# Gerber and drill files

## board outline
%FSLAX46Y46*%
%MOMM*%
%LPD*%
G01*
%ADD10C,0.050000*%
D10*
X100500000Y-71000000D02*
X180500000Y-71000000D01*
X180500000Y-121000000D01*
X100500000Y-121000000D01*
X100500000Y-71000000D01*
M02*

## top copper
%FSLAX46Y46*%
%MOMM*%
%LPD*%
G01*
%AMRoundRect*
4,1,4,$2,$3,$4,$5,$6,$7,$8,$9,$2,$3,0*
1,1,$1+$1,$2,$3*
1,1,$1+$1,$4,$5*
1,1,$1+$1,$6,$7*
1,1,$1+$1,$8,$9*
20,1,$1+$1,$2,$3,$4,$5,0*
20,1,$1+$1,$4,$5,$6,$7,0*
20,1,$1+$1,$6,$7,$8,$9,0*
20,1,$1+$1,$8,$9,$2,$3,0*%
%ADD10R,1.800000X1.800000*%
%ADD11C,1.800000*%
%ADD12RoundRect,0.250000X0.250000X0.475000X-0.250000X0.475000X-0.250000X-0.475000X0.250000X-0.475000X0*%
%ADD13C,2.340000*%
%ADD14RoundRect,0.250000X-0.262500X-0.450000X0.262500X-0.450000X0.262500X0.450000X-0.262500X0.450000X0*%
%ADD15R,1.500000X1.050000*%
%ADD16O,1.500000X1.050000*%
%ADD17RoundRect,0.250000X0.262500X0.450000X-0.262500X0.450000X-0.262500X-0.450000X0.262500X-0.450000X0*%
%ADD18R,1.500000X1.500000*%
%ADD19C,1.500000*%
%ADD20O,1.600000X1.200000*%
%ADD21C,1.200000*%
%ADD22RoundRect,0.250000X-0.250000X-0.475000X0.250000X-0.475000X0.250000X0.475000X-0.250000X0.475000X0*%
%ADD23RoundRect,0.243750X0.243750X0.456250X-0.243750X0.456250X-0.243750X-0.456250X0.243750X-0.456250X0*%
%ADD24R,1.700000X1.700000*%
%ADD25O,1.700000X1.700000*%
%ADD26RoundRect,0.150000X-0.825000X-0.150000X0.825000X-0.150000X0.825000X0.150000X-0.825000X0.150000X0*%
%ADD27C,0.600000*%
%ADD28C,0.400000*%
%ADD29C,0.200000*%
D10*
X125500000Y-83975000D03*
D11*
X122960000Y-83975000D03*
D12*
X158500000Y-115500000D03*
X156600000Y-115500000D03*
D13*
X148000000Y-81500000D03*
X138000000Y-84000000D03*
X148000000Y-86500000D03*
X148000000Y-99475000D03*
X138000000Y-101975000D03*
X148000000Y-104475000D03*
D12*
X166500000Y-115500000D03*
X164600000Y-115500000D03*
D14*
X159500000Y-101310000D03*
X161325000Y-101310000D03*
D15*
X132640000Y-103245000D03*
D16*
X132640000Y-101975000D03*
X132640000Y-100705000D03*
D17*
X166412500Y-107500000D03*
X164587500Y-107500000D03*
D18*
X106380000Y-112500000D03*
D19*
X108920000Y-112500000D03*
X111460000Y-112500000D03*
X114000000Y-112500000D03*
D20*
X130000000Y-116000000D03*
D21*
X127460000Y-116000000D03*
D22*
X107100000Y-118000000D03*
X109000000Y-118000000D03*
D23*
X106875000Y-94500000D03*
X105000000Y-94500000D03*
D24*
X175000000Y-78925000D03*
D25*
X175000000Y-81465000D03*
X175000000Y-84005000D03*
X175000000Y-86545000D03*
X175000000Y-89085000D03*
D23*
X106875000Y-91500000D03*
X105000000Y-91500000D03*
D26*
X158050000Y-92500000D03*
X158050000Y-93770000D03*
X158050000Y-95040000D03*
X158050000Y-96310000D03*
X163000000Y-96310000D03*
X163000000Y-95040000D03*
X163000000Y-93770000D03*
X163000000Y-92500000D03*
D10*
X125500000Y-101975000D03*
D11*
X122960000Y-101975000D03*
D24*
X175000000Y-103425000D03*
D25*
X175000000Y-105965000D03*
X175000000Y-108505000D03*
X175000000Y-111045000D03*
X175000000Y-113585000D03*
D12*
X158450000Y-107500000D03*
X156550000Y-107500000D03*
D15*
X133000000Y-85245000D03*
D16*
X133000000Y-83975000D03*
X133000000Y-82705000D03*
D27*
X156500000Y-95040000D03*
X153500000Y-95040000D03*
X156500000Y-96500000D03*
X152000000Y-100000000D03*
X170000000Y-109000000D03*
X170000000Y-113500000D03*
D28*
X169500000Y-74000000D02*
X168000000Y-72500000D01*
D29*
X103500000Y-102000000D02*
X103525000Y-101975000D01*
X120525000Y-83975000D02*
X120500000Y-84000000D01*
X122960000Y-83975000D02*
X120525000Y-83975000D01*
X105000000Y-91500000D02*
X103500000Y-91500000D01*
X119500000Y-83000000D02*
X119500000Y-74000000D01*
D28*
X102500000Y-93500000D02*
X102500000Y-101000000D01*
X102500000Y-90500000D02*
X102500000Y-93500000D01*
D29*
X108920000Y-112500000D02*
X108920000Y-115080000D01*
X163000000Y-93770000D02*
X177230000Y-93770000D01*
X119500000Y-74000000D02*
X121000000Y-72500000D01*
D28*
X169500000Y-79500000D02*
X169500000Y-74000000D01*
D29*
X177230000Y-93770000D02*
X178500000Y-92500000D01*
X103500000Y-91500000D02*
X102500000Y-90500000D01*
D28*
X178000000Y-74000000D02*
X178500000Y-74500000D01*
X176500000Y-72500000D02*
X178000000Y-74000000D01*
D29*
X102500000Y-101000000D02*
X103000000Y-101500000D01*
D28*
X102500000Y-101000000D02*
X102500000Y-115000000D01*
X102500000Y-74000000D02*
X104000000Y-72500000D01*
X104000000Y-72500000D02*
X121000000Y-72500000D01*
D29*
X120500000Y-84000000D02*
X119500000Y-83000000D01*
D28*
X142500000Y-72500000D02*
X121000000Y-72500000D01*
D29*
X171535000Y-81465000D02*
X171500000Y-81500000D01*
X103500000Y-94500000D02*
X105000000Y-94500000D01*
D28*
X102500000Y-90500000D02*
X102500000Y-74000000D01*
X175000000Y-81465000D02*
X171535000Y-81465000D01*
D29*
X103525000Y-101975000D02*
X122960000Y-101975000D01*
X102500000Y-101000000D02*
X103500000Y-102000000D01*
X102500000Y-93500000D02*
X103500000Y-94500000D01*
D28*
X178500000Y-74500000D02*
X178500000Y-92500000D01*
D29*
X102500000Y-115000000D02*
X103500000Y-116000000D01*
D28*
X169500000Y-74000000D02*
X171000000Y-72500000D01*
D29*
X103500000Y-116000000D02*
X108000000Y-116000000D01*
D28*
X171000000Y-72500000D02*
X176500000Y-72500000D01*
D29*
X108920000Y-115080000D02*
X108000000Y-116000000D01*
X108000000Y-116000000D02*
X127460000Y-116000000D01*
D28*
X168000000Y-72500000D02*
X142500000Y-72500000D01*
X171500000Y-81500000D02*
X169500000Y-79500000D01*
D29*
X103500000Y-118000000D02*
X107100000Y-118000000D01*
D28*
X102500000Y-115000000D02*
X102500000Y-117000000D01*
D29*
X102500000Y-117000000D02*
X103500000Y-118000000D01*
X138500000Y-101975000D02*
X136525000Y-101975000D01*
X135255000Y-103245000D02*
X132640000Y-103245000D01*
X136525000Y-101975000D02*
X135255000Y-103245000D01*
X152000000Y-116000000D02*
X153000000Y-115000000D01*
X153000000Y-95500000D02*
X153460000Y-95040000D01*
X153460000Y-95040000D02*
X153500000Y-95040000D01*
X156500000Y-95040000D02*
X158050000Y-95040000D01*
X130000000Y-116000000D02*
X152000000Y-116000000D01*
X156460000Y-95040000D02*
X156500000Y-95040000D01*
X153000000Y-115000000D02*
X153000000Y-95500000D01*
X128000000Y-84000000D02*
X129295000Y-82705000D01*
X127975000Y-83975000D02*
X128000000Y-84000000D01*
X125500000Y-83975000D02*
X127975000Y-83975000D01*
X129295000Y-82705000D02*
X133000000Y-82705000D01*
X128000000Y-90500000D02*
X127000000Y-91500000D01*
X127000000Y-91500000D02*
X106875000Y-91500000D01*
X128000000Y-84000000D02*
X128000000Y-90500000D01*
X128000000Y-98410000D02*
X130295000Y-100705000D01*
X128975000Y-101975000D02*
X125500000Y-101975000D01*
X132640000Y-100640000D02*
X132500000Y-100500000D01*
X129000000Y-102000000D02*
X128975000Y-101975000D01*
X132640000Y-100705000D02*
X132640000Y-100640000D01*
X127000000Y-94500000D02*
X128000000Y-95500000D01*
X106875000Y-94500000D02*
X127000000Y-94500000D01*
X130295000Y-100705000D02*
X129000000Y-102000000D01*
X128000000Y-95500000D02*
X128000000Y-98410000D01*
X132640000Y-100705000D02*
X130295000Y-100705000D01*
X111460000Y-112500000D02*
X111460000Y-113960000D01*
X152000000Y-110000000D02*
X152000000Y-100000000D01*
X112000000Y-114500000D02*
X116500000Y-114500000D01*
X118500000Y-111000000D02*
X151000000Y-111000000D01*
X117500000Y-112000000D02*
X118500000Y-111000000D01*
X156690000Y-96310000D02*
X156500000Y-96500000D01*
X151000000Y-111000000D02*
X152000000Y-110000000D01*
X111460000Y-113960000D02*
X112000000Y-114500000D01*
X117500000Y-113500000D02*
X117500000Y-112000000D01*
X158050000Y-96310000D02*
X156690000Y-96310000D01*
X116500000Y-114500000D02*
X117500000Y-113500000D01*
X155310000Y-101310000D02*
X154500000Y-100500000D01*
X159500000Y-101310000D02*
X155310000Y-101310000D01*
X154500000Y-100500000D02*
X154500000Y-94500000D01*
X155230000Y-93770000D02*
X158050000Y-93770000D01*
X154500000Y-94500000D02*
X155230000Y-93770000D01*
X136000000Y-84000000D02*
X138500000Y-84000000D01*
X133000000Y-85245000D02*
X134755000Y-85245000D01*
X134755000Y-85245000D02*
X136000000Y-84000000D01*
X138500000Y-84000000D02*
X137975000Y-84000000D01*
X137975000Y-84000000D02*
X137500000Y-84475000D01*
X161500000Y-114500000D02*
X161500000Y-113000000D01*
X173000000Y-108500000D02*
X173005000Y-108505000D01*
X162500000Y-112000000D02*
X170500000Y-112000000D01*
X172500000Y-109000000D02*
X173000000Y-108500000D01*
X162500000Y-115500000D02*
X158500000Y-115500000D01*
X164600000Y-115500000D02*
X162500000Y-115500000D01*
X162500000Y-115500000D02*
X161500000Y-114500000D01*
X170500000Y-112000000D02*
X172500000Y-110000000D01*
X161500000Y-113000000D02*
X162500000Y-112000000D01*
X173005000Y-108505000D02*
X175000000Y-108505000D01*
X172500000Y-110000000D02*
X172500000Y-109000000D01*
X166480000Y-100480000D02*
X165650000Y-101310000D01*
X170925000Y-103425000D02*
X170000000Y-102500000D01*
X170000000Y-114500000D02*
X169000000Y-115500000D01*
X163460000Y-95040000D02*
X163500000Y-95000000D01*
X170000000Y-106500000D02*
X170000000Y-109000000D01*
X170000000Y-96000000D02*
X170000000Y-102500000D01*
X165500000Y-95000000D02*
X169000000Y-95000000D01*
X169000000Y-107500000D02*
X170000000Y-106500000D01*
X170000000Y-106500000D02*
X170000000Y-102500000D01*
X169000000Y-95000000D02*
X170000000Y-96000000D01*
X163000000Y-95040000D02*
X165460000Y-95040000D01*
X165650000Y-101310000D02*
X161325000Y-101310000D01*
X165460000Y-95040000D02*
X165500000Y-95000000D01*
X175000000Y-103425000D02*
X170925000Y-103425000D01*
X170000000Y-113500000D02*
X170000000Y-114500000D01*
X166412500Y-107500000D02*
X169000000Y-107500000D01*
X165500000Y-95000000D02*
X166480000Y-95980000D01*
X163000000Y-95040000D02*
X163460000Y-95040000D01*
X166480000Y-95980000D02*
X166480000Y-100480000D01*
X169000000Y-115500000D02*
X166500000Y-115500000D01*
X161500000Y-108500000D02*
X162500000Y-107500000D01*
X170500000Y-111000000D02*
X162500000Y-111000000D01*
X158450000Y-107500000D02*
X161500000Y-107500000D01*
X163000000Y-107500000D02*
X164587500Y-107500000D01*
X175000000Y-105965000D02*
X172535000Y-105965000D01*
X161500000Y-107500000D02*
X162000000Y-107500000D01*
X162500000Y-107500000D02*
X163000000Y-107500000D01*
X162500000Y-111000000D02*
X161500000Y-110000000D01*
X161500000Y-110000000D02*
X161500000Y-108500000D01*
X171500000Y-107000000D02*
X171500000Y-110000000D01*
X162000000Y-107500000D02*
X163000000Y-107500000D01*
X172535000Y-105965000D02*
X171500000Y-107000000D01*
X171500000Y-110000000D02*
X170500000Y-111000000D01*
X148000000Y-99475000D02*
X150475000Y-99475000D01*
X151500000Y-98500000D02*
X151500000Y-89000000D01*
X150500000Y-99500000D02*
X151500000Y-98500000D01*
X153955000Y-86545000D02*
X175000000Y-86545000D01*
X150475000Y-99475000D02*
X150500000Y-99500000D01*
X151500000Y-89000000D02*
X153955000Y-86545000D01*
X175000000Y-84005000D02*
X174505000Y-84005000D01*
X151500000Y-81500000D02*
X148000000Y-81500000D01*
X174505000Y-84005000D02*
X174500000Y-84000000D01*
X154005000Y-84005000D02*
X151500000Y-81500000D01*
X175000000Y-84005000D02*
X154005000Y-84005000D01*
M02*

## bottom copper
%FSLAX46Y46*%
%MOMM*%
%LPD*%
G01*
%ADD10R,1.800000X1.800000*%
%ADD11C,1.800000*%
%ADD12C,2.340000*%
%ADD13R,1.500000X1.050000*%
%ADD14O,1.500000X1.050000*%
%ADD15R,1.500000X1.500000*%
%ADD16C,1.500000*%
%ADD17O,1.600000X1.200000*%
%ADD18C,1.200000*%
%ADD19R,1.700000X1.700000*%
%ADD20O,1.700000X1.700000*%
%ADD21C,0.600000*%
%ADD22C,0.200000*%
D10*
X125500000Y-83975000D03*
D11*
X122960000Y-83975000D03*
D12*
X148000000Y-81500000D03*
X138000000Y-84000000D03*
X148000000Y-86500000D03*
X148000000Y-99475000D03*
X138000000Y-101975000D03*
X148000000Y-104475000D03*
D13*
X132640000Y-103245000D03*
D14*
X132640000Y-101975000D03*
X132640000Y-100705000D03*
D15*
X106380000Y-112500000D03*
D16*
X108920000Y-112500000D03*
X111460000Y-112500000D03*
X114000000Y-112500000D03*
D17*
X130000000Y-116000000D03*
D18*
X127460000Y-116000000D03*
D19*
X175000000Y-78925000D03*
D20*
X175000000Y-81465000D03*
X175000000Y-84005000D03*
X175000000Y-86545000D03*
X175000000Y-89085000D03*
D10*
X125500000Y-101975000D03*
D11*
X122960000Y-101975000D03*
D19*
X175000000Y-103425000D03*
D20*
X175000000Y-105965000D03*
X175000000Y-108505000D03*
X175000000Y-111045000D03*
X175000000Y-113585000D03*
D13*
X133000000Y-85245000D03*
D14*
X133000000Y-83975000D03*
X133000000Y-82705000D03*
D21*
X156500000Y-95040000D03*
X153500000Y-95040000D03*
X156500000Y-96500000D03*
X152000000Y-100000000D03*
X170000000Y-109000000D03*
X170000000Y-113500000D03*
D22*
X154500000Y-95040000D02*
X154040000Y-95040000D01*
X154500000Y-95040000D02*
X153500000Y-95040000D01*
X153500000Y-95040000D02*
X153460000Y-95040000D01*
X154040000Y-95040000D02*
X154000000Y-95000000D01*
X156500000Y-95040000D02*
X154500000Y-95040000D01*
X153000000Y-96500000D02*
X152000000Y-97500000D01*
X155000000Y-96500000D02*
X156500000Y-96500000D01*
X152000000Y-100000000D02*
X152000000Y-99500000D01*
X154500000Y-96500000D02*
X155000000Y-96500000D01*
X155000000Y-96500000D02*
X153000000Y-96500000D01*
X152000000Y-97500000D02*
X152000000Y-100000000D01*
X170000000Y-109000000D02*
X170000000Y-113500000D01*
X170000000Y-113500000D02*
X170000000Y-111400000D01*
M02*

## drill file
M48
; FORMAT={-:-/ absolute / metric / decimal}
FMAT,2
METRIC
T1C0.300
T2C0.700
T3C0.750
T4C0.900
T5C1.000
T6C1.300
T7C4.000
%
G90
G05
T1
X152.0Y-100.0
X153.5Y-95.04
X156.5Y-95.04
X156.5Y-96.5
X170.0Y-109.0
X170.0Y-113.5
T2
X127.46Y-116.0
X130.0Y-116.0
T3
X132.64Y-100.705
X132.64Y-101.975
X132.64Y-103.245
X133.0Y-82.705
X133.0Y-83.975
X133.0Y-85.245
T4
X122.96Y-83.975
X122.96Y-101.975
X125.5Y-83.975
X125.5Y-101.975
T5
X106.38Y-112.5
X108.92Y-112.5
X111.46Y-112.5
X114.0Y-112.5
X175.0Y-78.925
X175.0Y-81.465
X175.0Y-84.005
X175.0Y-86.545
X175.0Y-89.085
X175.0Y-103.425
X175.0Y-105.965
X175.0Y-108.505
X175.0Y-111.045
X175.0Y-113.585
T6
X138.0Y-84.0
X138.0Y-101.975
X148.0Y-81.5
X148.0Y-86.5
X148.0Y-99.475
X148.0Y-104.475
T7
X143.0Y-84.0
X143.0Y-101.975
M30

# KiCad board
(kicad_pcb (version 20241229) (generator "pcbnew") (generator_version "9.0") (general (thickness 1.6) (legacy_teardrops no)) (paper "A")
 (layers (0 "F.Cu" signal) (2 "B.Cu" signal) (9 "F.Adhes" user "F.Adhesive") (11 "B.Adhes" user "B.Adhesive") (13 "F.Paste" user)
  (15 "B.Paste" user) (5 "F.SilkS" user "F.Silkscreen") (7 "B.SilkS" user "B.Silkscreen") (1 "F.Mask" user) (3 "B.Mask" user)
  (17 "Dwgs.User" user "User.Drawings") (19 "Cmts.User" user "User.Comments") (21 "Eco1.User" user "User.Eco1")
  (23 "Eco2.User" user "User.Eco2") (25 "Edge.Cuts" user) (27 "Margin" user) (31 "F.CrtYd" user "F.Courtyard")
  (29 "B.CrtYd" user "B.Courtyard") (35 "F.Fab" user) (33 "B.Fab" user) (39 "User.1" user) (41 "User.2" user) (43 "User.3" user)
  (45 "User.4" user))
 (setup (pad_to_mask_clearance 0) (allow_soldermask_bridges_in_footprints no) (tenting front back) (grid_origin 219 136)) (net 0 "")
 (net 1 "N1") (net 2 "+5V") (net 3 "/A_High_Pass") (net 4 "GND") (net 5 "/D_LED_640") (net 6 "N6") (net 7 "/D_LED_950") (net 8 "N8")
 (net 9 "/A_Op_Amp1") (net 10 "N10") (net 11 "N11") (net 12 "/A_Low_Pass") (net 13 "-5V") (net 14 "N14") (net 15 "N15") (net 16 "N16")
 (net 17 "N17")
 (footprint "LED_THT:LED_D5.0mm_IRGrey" (layer "F.Cu") (at 125.5 83.975 180)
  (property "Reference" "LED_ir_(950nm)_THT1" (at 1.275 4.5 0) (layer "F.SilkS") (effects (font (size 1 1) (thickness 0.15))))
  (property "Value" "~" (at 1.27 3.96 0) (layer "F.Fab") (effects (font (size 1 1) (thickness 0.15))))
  (pad "1" thru_hole rect (at 0 0 180) (size 1.8 1.8) (drill 0.9) (layers "*.Cu" "*.Mask") (remove_unused_layers no) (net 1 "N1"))
  (pad "2" thru_hole circle (at 2.54 0 180) (size 1.8 1.8) (drill 0.9) (layers "*.Cu" "*.Mask") (remove_unused_layers no) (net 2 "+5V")))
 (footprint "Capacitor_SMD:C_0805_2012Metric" (layer "F.Cu") (at 157.55 115.5 180)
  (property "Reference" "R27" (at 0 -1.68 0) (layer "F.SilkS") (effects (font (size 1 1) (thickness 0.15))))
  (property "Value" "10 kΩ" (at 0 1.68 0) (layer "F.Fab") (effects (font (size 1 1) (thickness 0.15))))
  (pad "1" smd roundrect (at -0.95 0 180) (size 1 1.45) (layers "F.Cu" "F.Mask" "F.Paste") (roundrect_rratio 0.25) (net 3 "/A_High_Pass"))
  (pad "2" smd roundrect (at 0.95 0 180) (size 1 1.45) (layers "F.Cu" "F.Mask" "F.Paste") (roundrect_rratio 0.25) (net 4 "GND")))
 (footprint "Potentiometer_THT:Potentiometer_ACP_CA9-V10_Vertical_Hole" (layer "F.Cu") (at 148 81.5 180)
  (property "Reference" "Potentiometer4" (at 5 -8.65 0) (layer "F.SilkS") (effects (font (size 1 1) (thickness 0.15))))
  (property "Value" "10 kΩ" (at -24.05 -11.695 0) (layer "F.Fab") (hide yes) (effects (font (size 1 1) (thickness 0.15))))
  (pad "" np_thru_hole circle (at 5 -2.5 180) (size 4 4) (drill 4) (layers "*.Cu" "*.Mask"))
  (pad "1" thru_hole circle (at 0 0 180) (size 2.34 2.34) (drill 1.3) (layers "*.Cu" "*.Mask") (remove_unused_layers no)
   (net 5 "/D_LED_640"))
  (pad "2" thru_hole circle (at 10 -2.5 180) (size 2.34 2.34) (drill 1.3) (layers "*.Cu" "*.Mask") (remove_unused_layers no) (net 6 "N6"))
  (pad "3" thru_hole circle (at 0 -5 180) (size 2.34 2.34) (drill 1.3) (layers "*.Cu" "*.Mask") (remove_unused_layers no) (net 4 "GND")))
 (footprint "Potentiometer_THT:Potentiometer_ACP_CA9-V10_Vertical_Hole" (layer "F.Cu") (at 148 99.475 180)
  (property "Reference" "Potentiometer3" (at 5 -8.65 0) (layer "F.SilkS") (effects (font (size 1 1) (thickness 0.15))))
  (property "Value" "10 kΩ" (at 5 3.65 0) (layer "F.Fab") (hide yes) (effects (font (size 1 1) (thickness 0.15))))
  (pad "" np_thru_hole circle (at 5 -2.5 180) (size 4 4) (drill 4) (layers "*.Cu" "*.Mask"))
  (pad "1" thru_hole circle (at 0 0 180) (size 2.34 2.34) (drill 1.3) (layers "*.Cu" "*.Mask") (remove_unused_layers no)
   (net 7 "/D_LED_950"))
  (pad "2" thru_hole circle (at 10 -2.5 180) (size 2.34 2.34) (drill 1.3) (layers "*.Cu" "*.Mask") (remove_unused_layers no) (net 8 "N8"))
  (pad "3" thru_hole circle (at 0 -5 180) (size 2.34 2.34) (drill 1.3) (layers "*.Cu" "*.Mask") (remove_unused_layers no) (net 4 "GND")))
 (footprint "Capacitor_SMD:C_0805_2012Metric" (layer "F.Cu") (at 165.55 115.5 180)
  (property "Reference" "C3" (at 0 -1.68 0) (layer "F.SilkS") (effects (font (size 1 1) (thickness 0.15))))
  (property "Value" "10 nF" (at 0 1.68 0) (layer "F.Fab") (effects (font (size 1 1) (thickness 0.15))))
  (pad "1" smd roundrect (at -0.95 0 180) (size 1 1.45) (layers "F.Cu" "F.Mask" "F.Paste") (roundrect_rratio 0.25) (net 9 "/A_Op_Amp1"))
  (pad "2" smd roundrect (at 0.95 0 180) (size 1 1.45) (layers "F.Cu" "F.Mask" "F.Paste") (roundrect_rratio 0.25) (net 3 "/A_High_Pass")))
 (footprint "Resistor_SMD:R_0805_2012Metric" (layer "F.Cu") (at 160.4125 101.31)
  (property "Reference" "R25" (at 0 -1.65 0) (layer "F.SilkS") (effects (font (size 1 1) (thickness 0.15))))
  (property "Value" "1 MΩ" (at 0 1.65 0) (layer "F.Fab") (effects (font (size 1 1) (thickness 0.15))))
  (pad "1" smd roundrect (at -0.9125 0) (size 1.025 1.4) (layers "F.Cu" "F.Mask" "F.Paste") (roundrect_rratio 0.243902) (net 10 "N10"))
  (pad "2" smd roundrect (at 0.9125 0) (size 1.025 1.4) (layers "F.Cu" "F.Mask" "F.Paste") (roundrect_rratio 0.243902) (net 9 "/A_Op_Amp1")))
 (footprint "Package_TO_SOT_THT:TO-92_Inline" (layer "F.Cu") (at 132.64 103.245 90)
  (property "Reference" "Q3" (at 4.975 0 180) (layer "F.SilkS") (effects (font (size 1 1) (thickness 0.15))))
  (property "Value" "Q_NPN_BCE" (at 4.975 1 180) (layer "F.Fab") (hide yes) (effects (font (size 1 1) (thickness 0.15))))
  (pad "1" thru_hole rect (at 0 0 90) (size 1.05 1.5) (drill 0.75) (layers "*.Cu" "*.Mask") (remove_unused_layers no) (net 8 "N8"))
  (pad "2" thru_hole oval (at 1.27 0 90) (size 1.05 1.5) (drill 0.75) (layers "*.Cu" "*.Mask") (remove_unused_layers no) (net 4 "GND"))
  (pad "3" thru_hole oval (at 2.54 0 90) (size 1.05 1.5) (drill 0.75) (layers "*.Cu" "*.Mask") (remove_unused_layers no) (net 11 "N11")))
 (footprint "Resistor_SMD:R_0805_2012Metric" (layer "F.Cu") (at 165.5 107.5 180)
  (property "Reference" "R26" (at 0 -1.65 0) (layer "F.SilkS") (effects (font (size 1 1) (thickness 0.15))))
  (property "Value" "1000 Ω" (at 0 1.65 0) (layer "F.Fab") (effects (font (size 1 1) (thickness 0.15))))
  (pad "1" smd roundrect (at -0.9125 0 180) (size 1.025 1.4) (layers "F.Cu" "F.Mask" "F.Paste") (roundrect_rratio 0.243902)
   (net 9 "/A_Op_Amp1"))
  (pad "2" smd roundrect (at 0.9125 0 180) (size 1.025 1.4) (layers "F.Cu" "F.Mask" "F.Paste") (roundrect_rratio 0.243902)
   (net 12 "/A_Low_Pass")))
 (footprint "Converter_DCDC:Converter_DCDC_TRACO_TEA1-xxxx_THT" (layer "F.Cu") (at 106.38 112.5 90)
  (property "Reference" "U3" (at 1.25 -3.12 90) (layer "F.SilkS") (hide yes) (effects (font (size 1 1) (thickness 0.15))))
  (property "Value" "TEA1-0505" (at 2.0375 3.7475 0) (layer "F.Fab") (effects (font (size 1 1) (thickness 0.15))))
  (pad "1" thru_hole rect (at 0 0 90) (size 1.5 1.5) (drill 1) (layers "*.Cu" "*.Mask") (remove_unused_layers no) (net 4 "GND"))
  (pad "2" thru_hole circle (at 0 2.54 90) (size 1.5 1.5) (drill 1) (layers "*.Cu" "*.Mask") (remove_unused_layers no) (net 2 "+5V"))
  (pad "3" thru_hole circle (at 0 5.08 90) (size 1.5 1.5) (drill 1) (layers "*.Cu" "*.Mask") (remove_unused_layers no) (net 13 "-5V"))
  (pad "4" thru_hole circle (at 0 7.62 90) (size 1.5 1.5) (drill 1) (layers "*.Cu" "*.Mask") (remove_unused_layers no) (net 4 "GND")))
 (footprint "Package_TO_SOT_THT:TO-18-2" (layer "F.Cu") (at 130 116 180)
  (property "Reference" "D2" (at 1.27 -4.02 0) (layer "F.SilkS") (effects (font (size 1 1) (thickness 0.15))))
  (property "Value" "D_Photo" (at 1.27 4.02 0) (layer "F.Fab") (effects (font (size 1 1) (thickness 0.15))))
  (pad "1" thru_hole oval (at 0 0 180) (size 1.6 1.2) (drill 0.7) (layers "*.Cu" "*.Mask") (remove_unused_layers no) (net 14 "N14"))
  (pad "2" thru_hole circle (at 2.54 0 180) (size 1.2 1.2) (drill 0.7) (layers "*.Cu" "*.Mask") (remove_unused_layers no) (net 2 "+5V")))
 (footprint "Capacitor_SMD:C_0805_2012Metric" (layer "F.Cu") (at 108.05 118)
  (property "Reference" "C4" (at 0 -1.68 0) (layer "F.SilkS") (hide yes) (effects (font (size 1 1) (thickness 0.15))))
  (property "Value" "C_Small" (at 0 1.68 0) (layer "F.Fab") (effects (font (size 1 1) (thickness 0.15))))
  (pad "1" smd roundrect (at -0.95 0) (size 1 1.45) (layers "F.Cu" "F.Mask" "F.Paste") (roundrect_rratio 0.25) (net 2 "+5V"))
  (pad "2" smd roundrect (at 0.95 0) (size 1 1.45) (layers "F.Cu" "F.Mask" "F.Paste") (roundrect_rratio 0.25) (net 4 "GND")))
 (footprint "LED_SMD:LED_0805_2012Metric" (layer "F.Cu") (at 105.9375 94.5 180)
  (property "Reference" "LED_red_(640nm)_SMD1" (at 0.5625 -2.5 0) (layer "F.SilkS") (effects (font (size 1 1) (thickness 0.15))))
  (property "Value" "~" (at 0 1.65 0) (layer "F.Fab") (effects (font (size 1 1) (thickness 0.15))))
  (pad "1" smd roundrect (at -0.9375 0 180) (size 0.975 1.4) (layers "F.Cu" "F.Mask" "F.Paste") (roundrect_rratio 0.25) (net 11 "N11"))
  (pad "2" smd roundrect (at 0.9375 0 180) (size 0.975 1.4) (layers "F.Cu" "F.Mask" "F.Paste") (roundrect_rratio 0.25) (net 2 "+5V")))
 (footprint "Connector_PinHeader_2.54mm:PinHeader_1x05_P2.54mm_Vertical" (layer "F.Cu") (at 175 78.925)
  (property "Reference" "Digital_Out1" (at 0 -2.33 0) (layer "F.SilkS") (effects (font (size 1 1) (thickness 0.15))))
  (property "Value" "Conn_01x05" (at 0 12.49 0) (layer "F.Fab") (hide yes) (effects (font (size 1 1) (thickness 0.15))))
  (pad "1" thru_hole rect (at 0 0) (size 1.7 1.7) (drill 1) (layers "*.Cu" "*.Mask") (remove_unused_layers no) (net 4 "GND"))
  (pad "2" thru_hole oval (at 0 2.54) (size 1.7 1.7) (drill 1) (layers "*.Cu" "*.Mask") (remove_unused_layers no) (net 2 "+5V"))
  (pad "3" thru_hole oval (at 0 5.08) (size 1.7 1.7) (drill 1) (layers "*.Cu" "*.Mask") (remove_unused_layers no) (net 5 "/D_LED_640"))
  (pad "4" thru_hole oval (at 0 7.62) (size 1.7 1.7) (drill 1) (layers "*.Cu" "*.Mask") (remove_unused_layers no) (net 7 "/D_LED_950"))
  (pad "5" thru_hole oval (at 0 10.16) (size 1.7 1.7) (drill 1) (layers "*.Cu" "*.Mask") (remove_unused_layers no) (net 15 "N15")))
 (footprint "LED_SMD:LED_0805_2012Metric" (layer "F.Cu") (at 105.9375 91.5 180)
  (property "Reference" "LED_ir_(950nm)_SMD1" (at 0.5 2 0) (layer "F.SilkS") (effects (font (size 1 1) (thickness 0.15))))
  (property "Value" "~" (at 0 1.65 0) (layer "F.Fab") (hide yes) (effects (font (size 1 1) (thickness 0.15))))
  (pad "1" smd roundrect (at -0.9375 0 180) (size 0.975 1.4) (layers "F.Cu" "F.Mask" "F.Paste") (roundrect_rratio 0.25) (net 1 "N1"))
  (pad "2" smd roundrect (at 0.9375 0 180) (size 0.975 1.4) (layers "F.Cu" "F.Mask" "F.Paste") (roundrect_rratio 0.25) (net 2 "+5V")))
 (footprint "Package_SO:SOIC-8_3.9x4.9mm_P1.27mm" (layer "F.Cu") (at 160.525 94.405)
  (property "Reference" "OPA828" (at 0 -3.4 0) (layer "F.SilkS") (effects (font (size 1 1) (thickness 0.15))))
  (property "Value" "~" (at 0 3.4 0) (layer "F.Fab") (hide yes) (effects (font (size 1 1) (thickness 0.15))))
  (pad "1" smd roundrect (at -2.475 -1.905) (size 1.95 0.6) (layers "F.Cu" "F.Mask" "F.Paste") (roundrect_rratio 0.25))
  (pad "2" smd roundrect (at -2.475 -0.635) (size 1.95 0.6) (layers "F.Cu" "F.Mask" "F.Paste") (roundrect_rratio 0.25) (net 10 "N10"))
  (pad "3" smd roundrect (at -2.475 0.635) (size 1.95 0.6) (layers "F.Cu" "F.Mask" "F.Paste") (roundrect_rratio 0.25) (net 14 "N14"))
  (pad "4" smd roundrect (at -2.475 1.905) (size 1.95 0.6) (layers "F.Cu" "F.Mask" "F.Paste") (roundrect_rratio 0.25) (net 13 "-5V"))
  (pad "5" smd roundrect (at 2.475 1.905) (size 1.95 0.6) (layers "F.Cu" "F.Mask" "F.Paste") (roundrect_rratio 0.25))
  (pad "6" smd roundrect (at 2.475 0.635) (size 1.95 0.6) (layers "F.Cu" "F.Mask" "F.Paste") (roundrect_rratio 0.25) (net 9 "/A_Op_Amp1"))
  (pad "7" smd roundrect (at 2.475 -0.635) (size 1.95 0.6) (layers "F.Cu" "F.Mask" "F.Paste") (roundrect_rratio 0.25) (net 2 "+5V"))
  (pad "8" smd roundrect (at 2.475 -1.905) (size 1.95 0.6) (layers "F.Cu" "F.Mask" "F.Paste") (roundrect_rratio 0.25)))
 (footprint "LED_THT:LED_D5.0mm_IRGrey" (layer "F.Cu") (at 125.5 101.975 180)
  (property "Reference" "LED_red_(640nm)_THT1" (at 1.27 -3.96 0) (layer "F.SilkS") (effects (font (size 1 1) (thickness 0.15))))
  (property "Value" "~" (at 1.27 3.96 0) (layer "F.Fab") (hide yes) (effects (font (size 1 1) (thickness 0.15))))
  (pad "1" thru_hole rect (at 0 0 180) (size 1.8 1.8) (drill 0.9) (layers "*.Cu" "*.Mask") (remove_unused_layers no) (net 11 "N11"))
  (pad "2" thru_hole circle (at 2.54 0 180) (size 1.8 1.8) (drill 0.9) (layers "*.Cu" "*.Mask") (remove_unused_layers no) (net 2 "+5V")))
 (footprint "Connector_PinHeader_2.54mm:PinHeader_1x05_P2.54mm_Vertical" (layer "F.Cu") (at 175 103.425)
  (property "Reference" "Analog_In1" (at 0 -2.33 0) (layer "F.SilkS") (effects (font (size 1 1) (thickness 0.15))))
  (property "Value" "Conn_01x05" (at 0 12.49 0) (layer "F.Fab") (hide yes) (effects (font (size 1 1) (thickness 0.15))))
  (pad "1" thru_hole rect (at 0 0) (size 1.7 1.7) (drill 1) (layers "*.Cu" "*.Mask") (remove_unused_layers no) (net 9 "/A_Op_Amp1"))
  (pad "2" thru_hole oval (at 0 2.54) (size 1.7 1.7) (drill 1) (layers "*.Cu" "*.Mask") (remove_unused_layers no) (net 12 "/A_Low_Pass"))
  (pad "3" thru_hole oval (at 0 5.08) (size 1.7 1.7) (drill 1) (layers "*.Cu" "*.Mask") (remove_unused_layers no) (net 3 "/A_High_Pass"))
  (pad "4" thru_hole oval (at 0 7.62) (size 1.7 1.7) (drill 1) (layers "*.Cu" "*.Mask") (remove_unused_layers no) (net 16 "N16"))
  (pad "5" thru_hole oval (at 0 10.16) (size 1.7 1.7) (drill 1) (layers "*.Cu" "*.Mask") (remove_unused_layers no) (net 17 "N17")))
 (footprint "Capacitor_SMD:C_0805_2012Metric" (layer "F.Cu") (at 157.5 107.5 180)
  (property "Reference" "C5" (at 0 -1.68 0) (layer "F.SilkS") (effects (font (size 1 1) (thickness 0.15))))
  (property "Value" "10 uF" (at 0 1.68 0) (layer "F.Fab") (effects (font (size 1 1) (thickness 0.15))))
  (pad "1" smd roundrect (at -0.95 0 180) (size 1 1.45) (layers "F.Cu" "F.Mask" "F.Paste") (roundrect_rratio 0.25) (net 12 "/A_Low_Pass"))
  (pad "2" smd roundrect (at 0.95 0 180) (size 1 1.45) (layers "F.Cu" "F.Mask" "F.Paste") (roundrect_rratio 0.25) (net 4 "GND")))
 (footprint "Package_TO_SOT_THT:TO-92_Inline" (layer "F.Cu") (at 133 85.245 90)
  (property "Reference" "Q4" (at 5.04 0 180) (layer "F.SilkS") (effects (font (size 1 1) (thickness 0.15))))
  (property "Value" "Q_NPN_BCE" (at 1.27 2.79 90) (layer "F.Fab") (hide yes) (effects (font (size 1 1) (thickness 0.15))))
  (pad "1" thru_hole rect (at 0 0 90) (size 1.05 1.5) (drill 0.75) (layers "*.Cu" "*.Mask") (remove_unused_layers no) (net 6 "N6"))
  (pad "2" thru_hole oval (at 1.27 0 90) (size 1.05 1.5) (drill 0.75) (layers "*.Cu" "*.Mask") (remove_unused_layers no) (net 4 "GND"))
  (pad "3" thru_hole oval (at 2.54 0 90) (size 1.05 1.5) (drill 0.75) (layers "*.Cu" "*.Mask") (remove_unused_layers no) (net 1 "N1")))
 (gr_rect (start 100.5 71) (end 180.5 121) (stroke (width 0.05) (type solid)) (fill no) (layer "Edge.Cuts"))
 (segment (start 169.5 74) (end 168 72.5) (width 0.4) (layer "F.Cu") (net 2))
 (segment (start 103.5 102) (end 103.525 101.975) (width 0.2) (layer "F.Cu") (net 2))
 (segment (start 120.525 83.975) (end 120.5 84) (width 0.2) (layer "F.Cu") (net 2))
 (segment (start 122.96 83.975) (end 120.525 83.975) (width 0.2) (layer "F.Cu") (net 2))
 (segment (start 105 91.5) (end 103.5 91.5) (width 0.2) (layer "F.Cu") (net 2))
 (segment (start 119.5 83) (end 119.5 74) (width 0.2) (layer "F.Cu") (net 2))
 (segment (start 102.5 93.5) (end 102.5 101) (width 0.4) (layer "F.Cu") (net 2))
 (segment (start 102.5 90.5) (end 102.5 93.5) (width 0.4) (layer "F.Cu") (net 2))
 (segment (start 108.92 112.5) (end 108.92 115.08) (width 0.2) (layer "F.Cu") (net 2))
 (segment (start 163 93.77) (end 177.23 93.77) (width 0.2) (layer "F.Cu") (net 2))
 (segment (start 119.5 74) (end 121 72.5) (width 0.2) (layer "F.Cu") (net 2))
 (segment (start 169.5 79.5) (end 169.5 74) (width 0.4) (layer "F.Cu") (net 2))
 (segment (start 177.23 93.77) (end 178.5 92.5) (width 0.2) (layer "F.Cu") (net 2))
 (segment (start 103.5 91.5) (end 102.5 90.5) (width 0.2) (layer "F.Cu") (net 2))
 (segment (start 178 74) (end 178.5 74.5) (width 0.4) (layer "F.Cu") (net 2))
 (segment (start 176.5 72.5) (end 178 74) (width 0.4) (layer "F.Cu") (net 2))
 (segment (start 102.5 101) (end 103 101.5) (width 0.2) (layer "F.Cu") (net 2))
 (segment (start 102.5 101) (end 102.5 115) (width 0.4) (layer "F.Cu") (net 2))
 (segment (start 102.5 74) (end 104 72.5) (width 0.4) (layer "F.Cu") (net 2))
 (segment (start 104 72.5) (end 121 72.5) (width 0.4) (layer "F.Cu") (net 2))
 (segment (start 120.5 84) (end 119.5 83) (width 0.2) (layer "F.Cu") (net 2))
 (segment (start 142.5 72.5) (end 121 72.5) (width 0.4) (layer "F.Cu") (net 2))
 (segment (start 171.535 81.465) (end 171.5 81.5) (width 0.2) (layer "F.Cu") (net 2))
 (segment (start 103.5 94.5) (end 105 94.5) (width 0.2) (layer "F.Cu") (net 2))
 (segment (start 102.5 90.5) (end 102.5 74) (width 0.4) (layer "F.Cu") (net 2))
 (segment (start 175 81.465) (end 171.535 81.465) (width 0.4) (layer "F.Cu") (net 2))
 (segment (start 103.525 101.975) (end 122.96 101.975) (width 0.2) (layer "F.Cu") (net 2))
 (segment (start 102.5 101) (end 103.5 102) (width 0.2) (layer "F.Cu") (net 2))
 (segment (start 102.5 93.5) (end 103.5 94.5) (width 0.2) (layer "F.Cu") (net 2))
 (segment (start 178.5 74.5) (end 178.5 92.5) (width 0.4) (layer "F.Cu") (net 2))
 (segment (start 102.5 115) (end 103.5 116) (width 0.2) (layer "F.Cu") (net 2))
 (segment (start 169.5 74) (end 171 72.5) (width 0.4) (layer "F.Cu") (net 2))
 (segment (start 103.5 116) (end 108 116) (width 0.2) (layer "F.Cu") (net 2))
 (segment (start 171 72.5) (end 176.5 72.5) (width 0.4) (layer "F.Cu") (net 2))
 (segment (start 108.92 115.08) (end 108 116) (width 0.2) (layer "F.Cu") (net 2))
 (segment (start 108 116) (end 127.46 116) (width 0.2) (layer "F.Cu") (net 2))
 (segment (start 168 72.5) (end 142.5 72.5) (width 0.4) (layer "F.Cu") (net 2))
 (segment (start 171.5 81.5) (end 169.5 79.5) (width 0.4) (layer "F.Cu") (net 2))
 (segment (start 103.5 118) (end 107.1 118) (width 0.2) (layer "F.Cu") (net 2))
 (segment (start 102.5 115) (end 102.5 117) (width 0.4) (layer "F.Cu") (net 2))
 (segment (start 102.5 117) (end 103.5 118) (width 0.2) (layer "F.Cu") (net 2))
 (segment (start 138.5 101.975) (end 136.525 101.975) (width 0.2) (layer "F.Cu") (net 8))
 (segment (start 135.255 103.245) (end 132.64 103.245) (width 0.2) (layer "F.Cu") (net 8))
 (segment (start 136.525 101.975) (end 135.255 103.245) (width 0.2) (layer "F.Cu") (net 8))
 (segment (start 152 116) (end 153 115) (width 0.2) (layer "F.Cu") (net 14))
 (segment (start 153 95.5) (end 153.46 95.04) (width 0.2) (layer "F.Cu") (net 14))
 (segment (start 153.46 95.04) (end 153.5 95.04) (width 0.2) (layer "F.Cu") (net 14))
 (segment (start 156.5 95.04) (end 158.05 95.04) (width 0.2) (layer "F.Cu") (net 14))
 (segment (start 130 116) (end 152 116) (width 0.2) (layer "F.Cu") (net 14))
 (segment (start 156.46 95.04) (end 156.5 95.04) (width 0.2) (layer "F.Cu") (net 14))
 (segment (start 153 115) (end 153 95.5) (width 0.2) (layer "F.Cu") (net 14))
 (via (at 156.5 95.04) (size 0.6) (drill 0.3) (layers "F.Cu" "B.Cu") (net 14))
 (via (at 153.5 95.04) (size 0.6) (drill 0.3) (layers "F.Cu" "B.Cu") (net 14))
 (segment (start 154.5 95.04) (end 154.04 95.04) (width 0.2) (layer "B.Cu") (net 14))
 (segment (start 154.5 95.04) (end 153.5 95.04) (width 0.2) (layer "B.Cu") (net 14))
 (segment (start 153.5 95.04) (end 153.46 95.04) (width 0.2) (layer "B.Cu") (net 14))
 (segment (start 154.04 95.04) (end 154 95) (width 0.2) (layer "B.Cu") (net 14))
 (segment (start 156.5 95.04) (end 154.5 95.04) (width 0.2) (layer "B.Cu") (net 14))
 (segment (start 128 84) (end 129.295 82.705) (width 0.2) (layer "F.Cu") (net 1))
 (segment (start 127.975 83.975) (end 128 84) (width 0.2) (layer "F.Cu") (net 1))
 (segment (start 125.5 83.975) (end 127.975 83.975) (width 0.2) (layer "F.Cu") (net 1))
 (segment (start 129.295 82.705) (end 133 82.705) (width 0.2) (layer "F.Cu") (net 1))
 (segment (start 128 90.5) (end 127 91.5) (width 0.2) (layer "F.Cu") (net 1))
 (segment (start 127 91.5) (end 106.875 91.5) (width 0.2) (layer "F.Cu") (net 1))
 (segment (start 128 84) (end 128 90.5) (width 0.2) (layer "F.Cu") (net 1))
 (segment (start 128 98.41) (end 130.295 100.705) (width 0.2) (layer "F.Cu") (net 11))
 (segment (start 128.975 101.975) (end 125.5 101.975) (width 0.2) (layer "F.Cu") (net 11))
 (segment (start 132.64 100.64) (end 132.5 100.5) (width 0.2) (layer "F.Cu") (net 11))
 (segment (start 129 102) (end 128.975 101.975) (width 0.2) (layer "F.Cu") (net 11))
 (segment (start 132.64 100.705) (end 132.64 100.64) (width 0.2) (layer "F.Cu") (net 11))
 (segment (start 127 94.5) (end 128 95.5) (width 0.2) (layer "F.Cu") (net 11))
 (segment (start 106.875 94.5) (end 127 94.5) (width 0.2) (layer "F.Cu") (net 11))
 (segment (start 130.295 100.705) (end 129 102) (width 0.2) (layer "F.Cu") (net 11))
 (segment (start 128 95.5) (end 128 98.41) (width 0.2) (layer "F.Cu") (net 11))
 (segment (start 132.64 100.705) (end 130.295 100.705) (width 0.2) (layer "F.Cu") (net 11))
 (segment (start 111.46 112.5) (end 111.46 113.96) (width 0.2) (layer "F.Cu") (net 13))
 (segment (start 152 110) (end 152 100) (width 0.2) (layer "F.Cu") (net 13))
 (segment (start 112 114.5) (end 116.5 114.5) (width 0.2) (layer "F.Cu") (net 13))
 (segment (start 118.5 111) (end 151 111) (width 0.2) (layer "F.Cu") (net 13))
 (segment (start 117.5 112) (end 118.5 111) (width 0.2) (layer "F.Cu") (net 13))
 (segment (start 156.69 96.31) (end 156.5 96.5) (width 0.2) (layer "F.Cu") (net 13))
 (segment (start 151 111) (end 152 110) (width 0.2) (layer "F.Cu") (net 13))
 (segment (start 111.46 113.96) (end 112 114.5) (width 0.2) (layer "F.Cu") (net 13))
 (segment (start 117.5 113.5) (end 117.5 112) (width 0.2) (layer "F.Cu") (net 13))
 (segment (start 158.05 96.31) (end 156.69 96.31) (width 0.2) (layer "F.Cu") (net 13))
 (segment (start 116.5 114.5) (end 117.5 113.5) (width 0.2) (layer "F.Cu") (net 13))
 (via (at 156.5 96.5) (size 0.6) (drill 0.3) (layers "F.Cu" "B.Cu") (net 13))
 (via (at 152 100) (size 0.6) (drill 0.3) (layers "F.Cu" "B.Cu") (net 13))
 (segment (start 153 96.5) (end 152 97.5) (width 0.2) (layer "B.Cu") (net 13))
 (segment (start 155 96.5) (end 156.5 96.5) (width 0.2) (layer "B.Cu") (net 13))
 (segment (start 152 100) (end 152 99.5) (width 0.2) (layer "B.Cu") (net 13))
 (segment (start 154.5 96.5) (end 155 96.5) (width 0.2) (layer "B.Cu") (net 13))
 (segment (start 155 96.5) (end 153 96.5) (width 0.2) (layer "B.Cu") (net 13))
 (segment (start 152 97.5) (end 152 100) (width 0.2) (layer "B.Cu") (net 13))
 (segment (start 155.31 101.31) (end 154.5 100.5) (width 0.2) (layer "F.Cu") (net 10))
 (segment (start 159.5 101.31) (end 155.31 101.31) (width 0.2) (layer "F.Cu") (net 10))
 (segment (start 154.5 100.5) (end 154.5 94.5) (width 0.2) (layer "F.Cu") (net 10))
 (segment (start 155.23 93.77) (end 158.05 93.77) (width 0.2) (layer "F.Cu") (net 10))
 (segment (start 154.5 94.5) (end 155.23 93.77) (width 0.2) (layer "F.Cu") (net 10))
 (segment (start 136 84) (end 138.5 84) (width 0.2) (layer "F.Cu") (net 6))
 (segment (start 133 85.245) (end 134.755 85.245) (width 0.2) (layer "F.Cu") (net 6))
 (segment (start 134.755 85.245) (end 136 84) (width 0.2) (layer "F.Cu") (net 6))
 (segment (start 138.5 84) (end 137.975 84) (width 0.2) (layer "F.Cu") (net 6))
 (segment (start 137.975 84) (end 137.5 84.475) (width 0.2) (layer "F.Cu") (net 6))
 (segment (start 161.5 114.5) (end 161.5 113) (width 0.2) (layer "F.Cu") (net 3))
 (segment (start 173 108.5) (end 173.005 108.505) (width 0.2) (layer "F.Cu") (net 3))
 (segment (start 162.5 112) (end 170.5 112) (width 0.2) (layer "F.Cu") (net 3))
 (segment (start 172.5 109) (end 173 108.5) (width 0.2) (layer "F.Cu") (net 3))
 (segment (start 162.5 115.5) (end 158.5 115.5) (width 0.2) (layer "F.Cu") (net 3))
 (segment (start 164.6 115.5) (end 162.5 115.5) (width 0.2) (layer "F.Cu") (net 3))
 (segment (start 162.5 115.5) (end 161.5 114.5) (width 0.2) (layer "F.Cu") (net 3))
 (segment (start 170.5 112) (end 172.5 110) (width 0.2) (layer "F.Cu") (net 3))
 (segment (start 161.5 113) (end 162.5 112) (width 0.2) (layer "F.Cu") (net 3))
 (segment (start 173.005 108.505) (end 175 108.505) (width 0.2) (layer "F.Cu") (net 3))
 (segment (start 172.5 110) (end 172.5 109) (width 0.2) (layer "F.Cu") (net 3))
 (segment (start 166.48 100.48) (end 165.65 101.31) (width 0.2) (layer "F.Cu") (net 9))
 (segment (start 170.925 103.425) (end 170 102.5) (width 0.2) (layer "F.Cu") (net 9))
 (segment (start 170 114.5) (end 169 115.5) (width 0.2) (layer "F.Cu") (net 9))
 (segment (start 163.46 95.04) (end 163.5 95) (width 0.2) (layer "F.Cu") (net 9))
 (segment (start 170 106.5) (end 170 109) (width 0.2) (layer "F.Cu") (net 9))
 (segment (start 170 96) (end 170 102.5) (width 0.2) (layer "F.Cu") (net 9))
 (segment (start 165.5 95) (end 169 95) (width 0.2) (layer "F.Cu") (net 9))
 (segment (start 169 107.5) (end 170 106.5) (width 0.2) (layer "F.Cu") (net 9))
 (segment (start 170 106.5) (end 170 102.5) (width 0.2) (layer "F.Cu") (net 9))
 (segment (start 169 95) (end 170 96) (width 0.2) (layer "F.Cu") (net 9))
 (segment (start 163 95.04) (end 165.46 95.04) (width 0.2) (layer "F.Cu") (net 9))
 (segment (start 165.65 101.31) (end 161.325 101.31) (width 0.2) (layer "F.Cu") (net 9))
 (segment (start 165.46 95.04) (end 165.5 95) (width 0.2) (layer "F.Cu") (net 9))
 (segment (start 175 103.425) (end 170.925 103.425) (width 0.2) (layer "F.Cu") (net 9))
 (segment (start 170 113.5) (end 170 114.5) (width 0.2) (layer "F.Cu") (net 9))
 (segment (start 166.4125 107.5) (end 169 107.5) (width 0.2) (layer "F.Cu") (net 9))
 (segment (start 165.5 95) (end 166.48 95.98) (width 0.2) (layer "F.Cu") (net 9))
 (segment (start 163 95.04) (end 163.46 95.04) (width 0.2) (layer "F.Cu") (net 9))
 (segment (start 166.48 95.98) (end 166.48 100.48) (width 0.2) (layer "F.Cu") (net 9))
 (segment (start 169 115.5) (end 166.5 115.5) (width 0.2) (layer "F.Cu") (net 9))
 (via (at 170 109) (size 0.6) (drill 0.3) (layers "F.Cu" "B.Cu") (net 9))
 (via (at 170 113.5) (size 0.6) (drill 0.3) (layers "F.Cu" "B.Cu") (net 9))
 (segment (start 170 109) (end 170 113.5) (width 0.2) (layer "B.Cu") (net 9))
 (segment (start 170 113.5) (end 170 111.4) (width 0.2) (layer "B.Cu") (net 9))
 (segment (start 161.5 108.5) (end 162.5 107.5) (width 0.2) (layer "F.Cu") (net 12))
 (segment (start 170.5 111) (end 162.5 111) (width 0.2) (layer "F.Cu") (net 12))
 (segment (start 158.45 107.5) (end 161.5 107.5) (width 0.2) (layer "F.Cu") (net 12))
 (segment (start 163 107.5) (end 164.5875 107.5) (width 0.2) (layer "F.Cu") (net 12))
 (segment (start 175 105.965) (end 172.535 105.965) (width 0.2) (layer "F.Cu") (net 12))
 (segment (start 161.5 107.5) (end 162 107.5) (width 0.2) (layer "F.Cu") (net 12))
 (segment (start 162.5 107.5) (end 163 107.5) (width 0.2) (layer "F.Cu") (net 12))
 (segment (start 162.5 111) (end 161.5 110) (width 0.2) (layer "F.Cu") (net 12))
 (segment (start 161.5 110) (end 161.5 108.5) (width 0.2) (layer "F.Cu") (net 12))
 (segment (start 171.5 107) (end 171.5 110) (width 0.2) (layer "F.Cu") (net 12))
 (segment (start 162 107.5) (end 163 107.5) (width 0.2) (layer "F.Cu") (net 12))
 (segment (start 172.535 105.965) (end 171.5 107) (width 0.2) (layer "F.Cu") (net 12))
 (segment (start 171.5 110) (end 170.5 111) (width 0.2) (layer "F.Cu") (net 12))
 (segment (start 148 99.475) (end 150.475 99.475) (width 0.2) (layer "F.Cu") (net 7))
 (segment (start 151.5 98.5) (end 151.5 89) (width 0.2) (layer "F.Cu") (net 7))
 (segment (start 150.5 99.5) (end 151.5 98.5) (width 0.2) (layer "F.Cu") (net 7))
 (segment (start 153.955 86.545) (end 175 86.545) (width 0.2) (layer "F.Cu") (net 7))
 (segment (start 150.475 99.475) (end 150.5 99.5) (width 0.2) (layer "F.Cu") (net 7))
 (segment (start 151.5 89) (end 153.955 86.545) (width 0.2) (layer "F.Cu") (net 7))
 (segment (start 175 84.005) (end 174.505 84.005) (width 0.2) (layer "F.Cu") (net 5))
 (segment (start 151.5 81.5) (end 148 81.5) (width 0.2) (layer "F.Cu") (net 5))
 (segment (start 174.505 84.005) (end 174.5 84) (width 0.2) (layer "F.Cu") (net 5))
 (segment (start 154.005 84.005) (end 151.5 81.5) (width 0.2) (layer "F.Cu") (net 5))
 (segment (start 175 84.005) (end 154.005 84.005) (width 0.2) (layer "F.Cu") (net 5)))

